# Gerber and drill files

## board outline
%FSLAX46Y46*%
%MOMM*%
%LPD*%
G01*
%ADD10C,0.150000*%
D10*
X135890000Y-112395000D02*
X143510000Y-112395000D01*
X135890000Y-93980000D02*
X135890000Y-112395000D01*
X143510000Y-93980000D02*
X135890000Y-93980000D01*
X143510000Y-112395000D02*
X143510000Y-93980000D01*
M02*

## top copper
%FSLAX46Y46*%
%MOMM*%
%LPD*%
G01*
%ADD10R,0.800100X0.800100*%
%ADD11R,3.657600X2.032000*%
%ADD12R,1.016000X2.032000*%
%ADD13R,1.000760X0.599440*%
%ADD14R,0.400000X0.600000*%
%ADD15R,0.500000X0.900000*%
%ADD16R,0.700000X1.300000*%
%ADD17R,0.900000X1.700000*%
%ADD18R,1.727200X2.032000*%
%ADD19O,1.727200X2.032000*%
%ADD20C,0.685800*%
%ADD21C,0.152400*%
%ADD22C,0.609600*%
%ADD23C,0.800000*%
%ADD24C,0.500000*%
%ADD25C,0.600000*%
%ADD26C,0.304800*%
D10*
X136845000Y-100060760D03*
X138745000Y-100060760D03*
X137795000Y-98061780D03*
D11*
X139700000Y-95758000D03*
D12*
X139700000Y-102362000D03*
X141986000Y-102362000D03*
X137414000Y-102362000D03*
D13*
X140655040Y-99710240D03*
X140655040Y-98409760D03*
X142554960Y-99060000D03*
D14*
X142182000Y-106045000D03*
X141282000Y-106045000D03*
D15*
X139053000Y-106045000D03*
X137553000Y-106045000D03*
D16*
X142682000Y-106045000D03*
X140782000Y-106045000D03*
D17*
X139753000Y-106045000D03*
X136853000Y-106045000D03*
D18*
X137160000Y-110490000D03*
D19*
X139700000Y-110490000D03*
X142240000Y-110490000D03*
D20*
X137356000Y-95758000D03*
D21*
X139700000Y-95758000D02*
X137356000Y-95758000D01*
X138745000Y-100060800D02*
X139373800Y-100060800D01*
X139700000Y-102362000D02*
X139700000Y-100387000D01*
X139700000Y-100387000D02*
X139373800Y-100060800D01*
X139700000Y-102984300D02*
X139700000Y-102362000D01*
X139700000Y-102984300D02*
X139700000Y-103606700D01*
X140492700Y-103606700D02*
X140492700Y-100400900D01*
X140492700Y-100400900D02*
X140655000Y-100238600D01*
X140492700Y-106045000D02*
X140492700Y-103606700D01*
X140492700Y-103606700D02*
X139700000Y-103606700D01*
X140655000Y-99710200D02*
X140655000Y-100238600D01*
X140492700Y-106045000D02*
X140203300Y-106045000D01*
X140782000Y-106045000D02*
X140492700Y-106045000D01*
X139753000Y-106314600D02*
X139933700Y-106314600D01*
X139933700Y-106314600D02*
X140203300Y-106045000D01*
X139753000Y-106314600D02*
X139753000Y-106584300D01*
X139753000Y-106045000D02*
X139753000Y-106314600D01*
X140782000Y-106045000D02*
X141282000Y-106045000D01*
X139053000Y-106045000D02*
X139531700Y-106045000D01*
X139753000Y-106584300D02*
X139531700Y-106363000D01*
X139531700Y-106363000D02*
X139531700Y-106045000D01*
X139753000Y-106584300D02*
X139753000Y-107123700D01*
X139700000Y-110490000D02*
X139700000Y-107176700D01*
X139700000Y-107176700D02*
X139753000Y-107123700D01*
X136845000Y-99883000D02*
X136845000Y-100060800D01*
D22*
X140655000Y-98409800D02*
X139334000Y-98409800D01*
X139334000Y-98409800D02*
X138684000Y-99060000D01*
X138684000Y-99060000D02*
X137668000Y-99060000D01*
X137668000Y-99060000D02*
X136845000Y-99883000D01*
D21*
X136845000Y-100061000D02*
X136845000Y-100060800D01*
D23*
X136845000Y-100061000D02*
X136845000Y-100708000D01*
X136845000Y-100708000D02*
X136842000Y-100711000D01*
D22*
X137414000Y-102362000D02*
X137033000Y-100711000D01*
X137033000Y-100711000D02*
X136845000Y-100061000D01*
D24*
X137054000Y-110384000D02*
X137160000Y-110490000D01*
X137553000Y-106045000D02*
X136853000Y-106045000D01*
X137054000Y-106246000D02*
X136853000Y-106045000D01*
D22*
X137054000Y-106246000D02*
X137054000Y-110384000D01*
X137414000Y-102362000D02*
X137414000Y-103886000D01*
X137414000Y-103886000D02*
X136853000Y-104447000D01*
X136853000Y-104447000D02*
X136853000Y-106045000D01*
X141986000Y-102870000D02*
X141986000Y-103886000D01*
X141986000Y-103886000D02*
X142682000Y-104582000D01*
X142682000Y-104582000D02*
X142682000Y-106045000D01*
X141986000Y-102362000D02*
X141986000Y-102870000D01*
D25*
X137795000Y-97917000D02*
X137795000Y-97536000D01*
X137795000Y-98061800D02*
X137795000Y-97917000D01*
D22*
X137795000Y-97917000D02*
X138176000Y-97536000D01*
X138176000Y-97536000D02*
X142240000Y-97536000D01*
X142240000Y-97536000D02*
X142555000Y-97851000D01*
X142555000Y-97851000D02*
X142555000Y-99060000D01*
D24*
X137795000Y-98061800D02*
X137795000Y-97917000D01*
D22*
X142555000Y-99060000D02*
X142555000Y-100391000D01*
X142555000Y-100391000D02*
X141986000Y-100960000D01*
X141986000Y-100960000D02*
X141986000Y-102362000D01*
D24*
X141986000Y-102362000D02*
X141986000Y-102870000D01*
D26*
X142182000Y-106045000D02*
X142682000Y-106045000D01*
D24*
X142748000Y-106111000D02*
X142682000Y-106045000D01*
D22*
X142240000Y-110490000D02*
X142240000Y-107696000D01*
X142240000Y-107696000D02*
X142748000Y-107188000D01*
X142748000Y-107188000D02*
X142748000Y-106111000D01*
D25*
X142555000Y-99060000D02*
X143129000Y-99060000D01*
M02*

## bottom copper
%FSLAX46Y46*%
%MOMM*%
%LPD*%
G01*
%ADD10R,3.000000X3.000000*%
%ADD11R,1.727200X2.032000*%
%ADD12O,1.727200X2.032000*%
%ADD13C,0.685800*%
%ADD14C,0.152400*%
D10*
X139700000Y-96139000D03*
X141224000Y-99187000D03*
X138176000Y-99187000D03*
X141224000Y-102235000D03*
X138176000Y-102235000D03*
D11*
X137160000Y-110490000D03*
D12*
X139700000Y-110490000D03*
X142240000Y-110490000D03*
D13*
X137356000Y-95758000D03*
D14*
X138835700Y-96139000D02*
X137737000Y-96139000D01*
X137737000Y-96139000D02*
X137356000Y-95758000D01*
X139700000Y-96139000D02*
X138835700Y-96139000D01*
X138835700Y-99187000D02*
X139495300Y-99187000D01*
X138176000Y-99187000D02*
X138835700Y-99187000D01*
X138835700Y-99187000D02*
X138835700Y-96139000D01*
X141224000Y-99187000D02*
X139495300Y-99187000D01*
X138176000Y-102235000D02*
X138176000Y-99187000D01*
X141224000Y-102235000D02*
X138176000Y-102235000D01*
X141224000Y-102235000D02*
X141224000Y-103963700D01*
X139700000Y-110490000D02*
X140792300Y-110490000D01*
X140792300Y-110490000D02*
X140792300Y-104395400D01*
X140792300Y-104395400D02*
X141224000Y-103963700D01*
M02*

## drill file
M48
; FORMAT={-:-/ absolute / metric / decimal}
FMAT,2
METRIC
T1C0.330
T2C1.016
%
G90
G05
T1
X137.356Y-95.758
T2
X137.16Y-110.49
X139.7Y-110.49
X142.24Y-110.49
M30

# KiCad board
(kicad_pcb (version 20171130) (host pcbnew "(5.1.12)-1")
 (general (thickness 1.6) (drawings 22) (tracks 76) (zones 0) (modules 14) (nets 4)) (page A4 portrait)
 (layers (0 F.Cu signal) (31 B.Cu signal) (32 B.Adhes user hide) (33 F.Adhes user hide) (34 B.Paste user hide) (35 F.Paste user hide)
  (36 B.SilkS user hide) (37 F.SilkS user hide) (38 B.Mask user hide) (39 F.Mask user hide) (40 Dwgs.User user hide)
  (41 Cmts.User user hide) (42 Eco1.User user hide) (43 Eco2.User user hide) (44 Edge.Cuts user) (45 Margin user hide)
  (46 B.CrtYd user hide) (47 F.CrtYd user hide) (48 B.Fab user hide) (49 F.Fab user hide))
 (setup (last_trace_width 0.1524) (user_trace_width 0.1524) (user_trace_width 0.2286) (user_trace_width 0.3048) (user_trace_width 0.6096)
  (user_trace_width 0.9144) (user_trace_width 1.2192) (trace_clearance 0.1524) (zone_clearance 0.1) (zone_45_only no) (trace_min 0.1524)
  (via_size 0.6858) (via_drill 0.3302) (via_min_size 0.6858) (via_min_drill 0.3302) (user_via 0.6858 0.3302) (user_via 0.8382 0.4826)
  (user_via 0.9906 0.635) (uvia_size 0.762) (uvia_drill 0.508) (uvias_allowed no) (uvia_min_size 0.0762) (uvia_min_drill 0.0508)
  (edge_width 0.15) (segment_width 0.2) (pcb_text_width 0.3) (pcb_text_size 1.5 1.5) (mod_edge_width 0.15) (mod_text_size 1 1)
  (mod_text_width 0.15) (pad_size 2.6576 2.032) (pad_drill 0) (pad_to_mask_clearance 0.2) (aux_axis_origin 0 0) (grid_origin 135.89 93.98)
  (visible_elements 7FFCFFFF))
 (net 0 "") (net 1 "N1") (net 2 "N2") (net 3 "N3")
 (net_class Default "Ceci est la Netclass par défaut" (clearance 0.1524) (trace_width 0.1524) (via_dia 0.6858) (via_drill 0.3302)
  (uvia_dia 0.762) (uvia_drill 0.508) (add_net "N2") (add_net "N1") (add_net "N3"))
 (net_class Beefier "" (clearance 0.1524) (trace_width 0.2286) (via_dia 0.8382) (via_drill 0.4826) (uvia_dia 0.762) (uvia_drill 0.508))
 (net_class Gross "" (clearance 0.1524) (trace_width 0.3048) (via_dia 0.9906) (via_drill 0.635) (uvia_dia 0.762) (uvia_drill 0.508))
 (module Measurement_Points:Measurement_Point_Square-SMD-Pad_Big (layer B.Cu) (at 139.7 96.139)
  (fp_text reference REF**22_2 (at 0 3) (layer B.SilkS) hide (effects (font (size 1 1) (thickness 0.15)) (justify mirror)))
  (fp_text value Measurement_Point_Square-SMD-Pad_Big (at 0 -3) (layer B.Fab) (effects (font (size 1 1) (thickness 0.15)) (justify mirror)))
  (pad 1 smd rect (at 0 0) (size 3 3) (layers B.Cu B.Mask) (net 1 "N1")))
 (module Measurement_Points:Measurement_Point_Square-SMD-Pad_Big (layer B.Cu) (at 141.224 99.187)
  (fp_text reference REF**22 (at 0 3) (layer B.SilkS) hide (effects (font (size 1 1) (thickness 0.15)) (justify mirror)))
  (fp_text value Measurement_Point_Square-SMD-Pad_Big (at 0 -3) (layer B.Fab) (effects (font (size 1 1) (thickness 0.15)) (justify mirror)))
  (pad 1 smd rect (at 0 0) (size 3 3) (layers B.Cu B.Mask) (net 1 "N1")))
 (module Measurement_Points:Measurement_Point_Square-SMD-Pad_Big (layer B.Cu) (at 138.176 99.187) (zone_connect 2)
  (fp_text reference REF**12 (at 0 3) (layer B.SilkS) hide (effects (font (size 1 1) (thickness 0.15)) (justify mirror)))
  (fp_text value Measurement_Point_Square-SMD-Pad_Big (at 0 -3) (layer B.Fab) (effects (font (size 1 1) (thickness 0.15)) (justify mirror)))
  (pad 1 smd rect (at 0 0) (size 3 3) (layers B.Cu B.Mask) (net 1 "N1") (zone_connect 2)))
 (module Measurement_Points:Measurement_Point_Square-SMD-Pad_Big (layer B.Cu) (at 141.224 102.235)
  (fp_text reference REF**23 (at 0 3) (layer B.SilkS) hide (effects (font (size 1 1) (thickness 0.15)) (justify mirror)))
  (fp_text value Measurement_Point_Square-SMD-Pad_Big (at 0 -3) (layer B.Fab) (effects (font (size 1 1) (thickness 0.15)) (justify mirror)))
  (pad 1 smd rect (at 0 0) (size 3 3) (layers B.Cu B.Mask) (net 1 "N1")))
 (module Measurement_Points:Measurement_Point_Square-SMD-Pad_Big (layer B.Cu) (at 138.176 102.235) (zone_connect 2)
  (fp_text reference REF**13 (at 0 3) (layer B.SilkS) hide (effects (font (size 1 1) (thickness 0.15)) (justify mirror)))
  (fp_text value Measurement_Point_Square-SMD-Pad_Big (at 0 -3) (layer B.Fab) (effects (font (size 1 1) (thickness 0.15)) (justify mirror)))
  (pad 1 smd rect (at 0 0) (size 3 3) (layers B.Cu B.Mask) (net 1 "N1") (zone_connect 2)))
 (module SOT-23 (layer F.Cu) (at 137.795 99.06)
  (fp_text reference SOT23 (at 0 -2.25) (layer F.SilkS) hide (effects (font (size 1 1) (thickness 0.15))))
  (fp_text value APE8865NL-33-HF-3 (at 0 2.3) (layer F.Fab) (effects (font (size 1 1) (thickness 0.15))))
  (pad 1 smd rect (at -0.95 1.00076) (size 0.8001 0.8001) (layers F.Cu F.Paste F.Mask) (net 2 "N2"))
  (pad 2 smd rect (at 0.95 1.00076) (size 0.8001 0.8001) (layers F.Cu F.Paste F.Mask) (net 1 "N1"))
  (pad 3 smd rect (at 0 -0.99822) (size 0.8001 0.8001) (layers F.Cu F.Paste F.Mask) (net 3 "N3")))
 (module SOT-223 (layer F.Cu) (at 139.7 99.06)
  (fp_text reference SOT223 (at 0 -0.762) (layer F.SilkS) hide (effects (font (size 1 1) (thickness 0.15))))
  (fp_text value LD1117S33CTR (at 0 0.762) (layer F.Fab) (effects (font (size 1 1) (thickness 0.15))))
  (pad 4 smd rect (at 0 -3.302) (size 3.6576 2.032) (layers F.Cu F.Paste F.Mask) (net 1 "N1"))
  (pad 2 smd rect (at 0 3.302) (size 1.016 2.032) (layers F.Cu F.Paste F.Mask) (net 1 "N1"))
  (pad 3 smd rect (at 2.286 3.302) (size 1.016 2.032) (layers F.Cu F.Paste F.Mask) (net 3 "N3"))
  (pad 1 smd rect (at -2.286 3.302) (size 1.016 2.032) (layers F.Cu F.Paste F.Mask) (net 2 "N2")))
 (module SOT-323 (layer F.Cu) (at 141.605 99.06 90)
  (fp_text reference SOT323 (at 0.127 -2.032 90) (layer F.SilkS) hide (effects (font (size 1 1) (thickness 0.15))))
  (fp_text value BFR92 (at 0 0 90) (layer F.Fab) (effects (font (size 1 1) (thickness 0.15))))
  (pad 2 smd rect (at -0.65024 -0.94996 90) (size 0.59944 1.00076) (layers F.Cu F.Paste F.Mask) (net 1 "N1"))
  (pad 1 smd rect (at 0.65024 -0.94996 90) (size 0.59944 1.00076) (layers F.Cu F.Paste F.Mask) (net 2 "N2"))
  (pad 3 smd rect (at 0 0.94996 90) (size 0.59944 1.00076) (layers F.Cu F.Paste F.Mask) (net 3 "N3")))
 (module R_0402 (layer F.Cu) (at 141.732 106.045 180)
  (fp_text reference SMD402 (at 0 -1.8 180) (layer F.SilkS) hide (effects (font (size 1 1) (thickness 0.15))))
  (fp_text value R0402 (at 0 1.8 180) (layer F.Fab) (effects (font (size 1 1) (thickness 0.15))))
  (pad 1 smd rect (at -0.45 0 180) (size 0.4 0.6) (layers F.Cu F.Paste F.Mask) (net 3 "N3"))
  (pad 2 smd rect (at 0.45 0 180) (size 0.4 0.6) (layers F.Cu F.Paste F.Mask) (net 1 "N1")))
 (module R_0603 (layer F.Cu) (at 138.303 106.045 180)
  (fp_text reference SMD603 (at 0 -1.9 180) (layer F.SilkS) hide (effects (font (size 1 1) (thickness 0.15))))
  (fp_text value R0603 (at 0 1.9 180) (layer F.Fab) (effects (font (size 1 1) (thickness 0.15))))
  (pad 1 smd rect (at -0.75 0 180) (size 0.5 0.9) (layers F.Cu F.Paste F.Mask) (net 1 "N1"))
  (pad 2 smd rect (at 0.75 0 180) (size 0.5 0.9) (layers F.Cu F.Paste F.Mask) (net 2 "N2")))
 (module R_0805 (layer F.Cu) (at 141.732 106.045 180)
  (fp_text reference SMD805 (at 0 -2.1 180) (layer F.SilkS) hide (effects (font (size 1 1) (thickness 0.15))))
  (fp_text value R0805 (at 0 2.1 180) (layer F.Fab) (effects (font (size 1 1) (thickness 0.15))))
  (pad 1 smd rect (at -0.95 0 180) (size 0.7 1.3) (layers F.Cu F.Paste F.Mask) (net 3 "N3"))
  (pad 2 smd rect (at 0.95 0 180) (size 0.7 1.3) (layers F.Cu F.Paste F.Mask) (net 1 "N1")))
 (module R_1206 (layer F.Cu) (at 138.303 106.045 180)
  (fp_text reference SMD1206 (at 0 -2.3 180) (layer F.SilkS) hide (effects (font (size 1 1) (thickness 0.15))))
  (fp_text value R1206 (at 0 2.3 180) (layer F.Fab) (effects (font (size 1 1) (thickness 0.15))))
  (pad 1 smd rect (at -1.45 0 180) (size 0.9 1.7) (layers F.Cu F.Paste F.Mask) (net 1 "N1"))
  (pad 2 smd rect (at 1.45 0 180) (size 0.9 1.7) (layers F.Cu F.Paste F.Mask) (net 2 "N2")))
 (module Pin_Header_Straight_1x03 (layer F.Cu) (at 137.16 110.49 90)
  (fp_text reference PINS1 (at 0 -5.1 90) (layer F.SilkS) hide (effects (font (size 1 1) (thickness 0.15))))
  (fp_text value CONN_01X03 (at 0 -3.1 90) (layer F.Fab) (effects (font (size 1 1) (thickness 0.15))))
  (pad 1 thru_hole rect (at 0 0 90) (size 2.032 1.7272) (drill 1.016) (layers *.Cu *.Mask F.SilkS) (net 2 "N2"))
  (pad 2 thru_hole oval (at 0 2.54 90) (size 2.032 1.7272) (drill 1.016) (layers *.Cu *.Mask F.SilkS) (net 1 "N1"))
  (pad 3 thru_hole oval (at 0 5.08 90) (size 2.032 1.7272) (drill 1.016) (layers *.Cu *.Mask F.SilkS) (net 3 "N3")))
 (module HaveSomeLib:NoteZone (layer B.Cu) (at 139.7 108.204)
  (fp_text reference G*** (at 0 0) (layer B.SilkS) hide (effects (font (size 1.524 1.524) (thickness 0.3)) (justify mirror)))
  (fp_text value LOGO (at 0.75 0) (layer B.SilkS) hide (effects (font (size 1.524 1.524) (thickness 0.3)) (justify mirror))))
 (gr_line (start 135.89 112.395) (end 143.51 112.395) (angle 90) (layer Edge.Cuts) (width 0.15))
 (gr_line (start 135.89 93.98) (end 135.89 112.395) (angle 90) (layer Edge.Cuts) (width 0.15))
 (gr_line (start 143.51 93.98) (end 135.89 93.98) (angle 90) (layer Edge.Cuts) (width 0.15))
 (gr_line (start 143.51 112.395) (end 143.51 93.98) (angle 90) (layer Edge.Cuts) (width 0.15))
 (segment (start 138.8357 96.139) (end 137.737 96.139) (width 0.1524) (layer B.Cu) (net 1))
 (segment (start 137.737 96.139) (end 137.356 95.758) (width 0.1524) (layer B.Cu) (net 1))
 (segment (start 139.7 96.139) (end 138.8357 96.139) (width 0.1524) (layer B.Cu) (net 1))
 (segment (start 138.8357 99.187) (end 139.4953 99.187) (width 0.1524) (layer B.Cu) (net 1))
 (segment (start 138.176 99.187) (end 138.8357 99.187) (width 0.1524) (layer B.Cu) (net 1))
 (segment (start 138.8357 99.187) (end 138.8357 96.139) (width 0.1524) (layer B.Cu) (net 1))
 (segment (start 141.224 99.187) (end 139.4953 99.187) (width 0.1524) (layer B.Cu) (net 1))
 (segment (start 138.176 102.235) (end 138.176 99.187) (width 0.1524) (layer B.Cu) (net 1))
 (segment (start 141.224 102.235) (end 138.176 102.235) (width 0.1524) (layer B.Cu) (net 1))
 (segment (start 141.224 102.235) (end 141.224 103.9637) (width 0.1524) (layer B.Cu) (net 1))
 (segment (start 139.7 110.49) (end 140.7923 110.49) (width 0.1524) (layer B.Cu) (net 1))
 (segment (start 140.7923 110.49) (end 140.7923 104.3954) (width 0.1524) (layer B.Cu) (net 1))
 (segment (start 140.7923 104.3954) (end 141.224 103.9637) (width 0.1524) (layer B.Cu) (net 1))
 (segment (start 139.7 95.758) (end 137.356 95.758) (width 0.1524) (layer F.Cu) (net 1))
 (segment (start 138.745 100.0608) (end 139.3738 100.0608) (width 0.1524) (layer F.Cu) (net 1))
 (segment (start 139.7 102.362) (end 139.7 100.387) (width 0.1524) (layer F.Cu) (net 1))
 (segment (start 139.7 100.387) (end 139.3738 100.0608) (width 0.1524) (layer F.Cu) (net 1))
 (segment (start 139.7 102.9843) (end 139.7 102.362) (width 0.1524) (layer F.Cu) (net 1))
 (segment (start 139.7 102.9843) (end 139.7 103.6067) (width 0.1524) (layer F.Cu) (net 1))
 (segment (start 140.4927 103.6067) (end 140.4927 100.4009) (width 0.1524) (layer F.Cu) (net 1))
 (segment (start 140.4927 100.4009) (end 140.655 100.2386) (width 0.1524) (layer F.Cu) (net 1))
 (segment (start 140.4927 106.045) (end 140.4927 103.6067) (width 0.1524) (layer F.Cu) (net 1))
 (segment (start 140.4927 103.6067) (end 139.7 103.6067) (width 0.1524) (layer F.Cu) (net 1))
 (segment (start 140.655 99.7102) (end 140.655 100.2386) (width 0.1524) (layer F.Cu) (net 1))
 (segment (start 140.4927 106.045) (end 140.2033 106.045) (width 0.1524) (layer F.Cu) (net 1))
 (segment (start 140.782 106.045) (end 140.4927 106.045) (width 0.1524) (layer F.Cu) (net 1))
 (segment (start 139.753 106.3146) (end 139.9337 106.3146) (width 0.1524) (layer F.Cu) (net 1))
 (segment (start 139.9337 106.3146) (end 140.2033 106.045) (width 0.1524) (layer F.Cu) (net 1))
 (segment (start 139.753 106.3146) (end 139.753 106.5843) (width 0.1524) (layer F.Cu) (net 1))
 (segment (start 139.753 106.045) (end 139.753 106.3146) (width 0.1524) (layer F.Cu) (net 1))
 (segment (start 140.782 106.045) (end 141.282 106.045) (width 0.1524) (layer F.Cu) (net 1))
 (segment (start 139.053 106.045) (end 139.5317 106.045) (width 0.1524) (layer F.Cu) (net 1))
 (segment (start 139.753 106.5843) (end 139.5317 106.363) (width 0.1524) (layer F.Cu) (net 1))
 (segment (start 139.5317 106.363) (end 139.5317 106.045) (width 0.1524) (layer F.Cu) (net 1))
 (segment (start 139.753 106.5843) (end 139.753 107.1237) (width 0.1524) (layer F.Cu) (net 1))
 (segment (start 139.7 110.49) (end 139.7 107.1767) (width 0.1524) (layer F.Cu) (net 1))
 (segment (start 139.7 107.1767) (end 139.753 107.1237) (width 0.1524) (layer F.Cu) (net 1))
 (via (at 137.356 95.758) (size 0.6858) (layers F.Cu B.Cu) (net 1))
 (segment (start 136.845 99.883) (end 136.845 100.0608) (width 0.1524) (layer F.Cu) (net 2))
 (segment (start 140.655 98.4098) (end 139.334 98.4098) (width 0.6096) (layer F.Cu) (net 2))
 (segment (start 139.334 98.4098) (end 138.684 99.06) (width 0.6096) (layer F.Cu) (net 2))
 (segment (start 138.684 99.06) (end 137.668 99.06) (width 0.6096) (layer F.Cu) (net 2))
 (segment (start 137.668 99.06) (end 136.845 99.883) (width 0.6096) (layer F.Cu) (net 2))
 (segment (start 136.845 100.061) (end 136.845 100.0608) (width 0.1524) (layer F.Cu) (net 2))
 (segment (start 136.845 100.061) (end 136.845 100.708) (width 0.8) (layer F.Cu) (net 2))
 (segment (start 136.845 100.708) (end 136.842 100.711) (width 0.8) (layer F.Cu) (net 2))
 (segment (start 137.414 102.362) (end 137.033 100.711) (width 0.6096) (layer F.Cu) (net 2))
 (segment (start 137.033 100.711) (end 136.845 100.061) (width 0.6096) (layer F.Cu) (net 2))
 (segment (start 137.054 110.384) (end 137.16 110.49) (width 0.5) (layer F.Cu) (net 2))
 (segment (start 137.553 106.045) (end 136.853 106.045) (width 0.5) (layer F.Cu) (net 2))
 (segment (start 137.054 106.246) (end 136.853 106.045) (width 0.5) (layer F.Cu) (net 2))
 (segment (start 137.054 106.246) (end 137.054 110.384) (width 0.6096) (layer F.Cu) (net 2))
 (segment (start 137.414 102.362) (end 137.414 103.886) (width 0.6096) (layer F.Cu) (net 2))
 (segment (start 137.414 103.886) (end 136.853 104.447) (width 0.6096) (layer F.Cu) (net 2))
 (segment (start 136.853 104.447) (end 136.853 106.045) (width 0.6096) (layer F.Cu) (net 2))
 (segment (start 141.986 102.87) (end 141.986 103.886) (width 0.6096) (layer F.Cu) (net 3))
 (segment (start 141.986 103.886) (end 142.682 104.582) (width 0.6096) (layer F.Cu) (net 3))
 (segment (start 142.682 104.582) (end 142.682 106.045) (width 0.6096) (layer F.Cu) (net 3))
 (segment (start 141.986 102.362) (end 141.986 102.87) (width 0.6096) (layer F.Cu) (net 3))
 (segment (start 137.795 97.917) (end 137.795 97.536) (width 0.6) (layer F.Cu) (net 3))
 (segment (start 137.795 98.0618) (end 137.795 97.917) (width 0.6) (layer F.Cu) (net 3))
 (segment (start 137.795 97.917) (end 138.176 97.536) (width 0.6096) (layer F.Cu) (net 3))
 (segment (start 138.176 97.536) (end 142.24 97.536) (width 0.6096) (layer F.Cu) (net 3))
 (segment (start 142.24 97.536) (end 142.555 97.851) (width 0.6096) (layer F.Cu) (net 3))
 (segment (start 142.555 97.851) (end 142.555 99.06) (width 0.6096) (layer F.Cu) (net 3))
 (segment (start 137.795 98.0618) (end 137.795 97.917) (width 0.5) (layer F.Cu) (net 3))
 (segment (start 142.555 99.06) (end 142.555 100.391) (width 0.6096) (layer F.Cu) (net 3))
 (segment (start 142.555 100.391) (end 141.986 100.96) (width 0.6096) (layer F.Cu) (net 3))
 (segment (start 141.986 100.96) (end 141.986 102.362) (width 0.6096) (layer F.Cu) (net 3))
 (segment (start 141.986 102.362) (end 141.986 102.87) (width 0.5) (layer F.Cu) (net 3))
 (segment (start 142.182 106.045) (end 142.682 106.045) (width 0.3048) (layer F.Cu) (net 3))
 (segment (start 142.748 106.111) (end 142.682 106.045) (width 0.5) (layer F.Cu) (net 3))
 (segment (start 142.24 110.49) (end 142.24 107.696) (width 0.6096) (layer F.Cu) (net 3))
 (segment (start 142.24 107.696) (end 142.748 107.188) (width 0.6096) (layer F.Cu) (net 3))
 (segment (start 142.748 107.188) (end 142.748 106.111) (width 0.6096) (layer F.Cu) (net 3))
 (segment (start 142.555 99.06) (end 143.129 99.06) (width 0.6) (layer F.Cu) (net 3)))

